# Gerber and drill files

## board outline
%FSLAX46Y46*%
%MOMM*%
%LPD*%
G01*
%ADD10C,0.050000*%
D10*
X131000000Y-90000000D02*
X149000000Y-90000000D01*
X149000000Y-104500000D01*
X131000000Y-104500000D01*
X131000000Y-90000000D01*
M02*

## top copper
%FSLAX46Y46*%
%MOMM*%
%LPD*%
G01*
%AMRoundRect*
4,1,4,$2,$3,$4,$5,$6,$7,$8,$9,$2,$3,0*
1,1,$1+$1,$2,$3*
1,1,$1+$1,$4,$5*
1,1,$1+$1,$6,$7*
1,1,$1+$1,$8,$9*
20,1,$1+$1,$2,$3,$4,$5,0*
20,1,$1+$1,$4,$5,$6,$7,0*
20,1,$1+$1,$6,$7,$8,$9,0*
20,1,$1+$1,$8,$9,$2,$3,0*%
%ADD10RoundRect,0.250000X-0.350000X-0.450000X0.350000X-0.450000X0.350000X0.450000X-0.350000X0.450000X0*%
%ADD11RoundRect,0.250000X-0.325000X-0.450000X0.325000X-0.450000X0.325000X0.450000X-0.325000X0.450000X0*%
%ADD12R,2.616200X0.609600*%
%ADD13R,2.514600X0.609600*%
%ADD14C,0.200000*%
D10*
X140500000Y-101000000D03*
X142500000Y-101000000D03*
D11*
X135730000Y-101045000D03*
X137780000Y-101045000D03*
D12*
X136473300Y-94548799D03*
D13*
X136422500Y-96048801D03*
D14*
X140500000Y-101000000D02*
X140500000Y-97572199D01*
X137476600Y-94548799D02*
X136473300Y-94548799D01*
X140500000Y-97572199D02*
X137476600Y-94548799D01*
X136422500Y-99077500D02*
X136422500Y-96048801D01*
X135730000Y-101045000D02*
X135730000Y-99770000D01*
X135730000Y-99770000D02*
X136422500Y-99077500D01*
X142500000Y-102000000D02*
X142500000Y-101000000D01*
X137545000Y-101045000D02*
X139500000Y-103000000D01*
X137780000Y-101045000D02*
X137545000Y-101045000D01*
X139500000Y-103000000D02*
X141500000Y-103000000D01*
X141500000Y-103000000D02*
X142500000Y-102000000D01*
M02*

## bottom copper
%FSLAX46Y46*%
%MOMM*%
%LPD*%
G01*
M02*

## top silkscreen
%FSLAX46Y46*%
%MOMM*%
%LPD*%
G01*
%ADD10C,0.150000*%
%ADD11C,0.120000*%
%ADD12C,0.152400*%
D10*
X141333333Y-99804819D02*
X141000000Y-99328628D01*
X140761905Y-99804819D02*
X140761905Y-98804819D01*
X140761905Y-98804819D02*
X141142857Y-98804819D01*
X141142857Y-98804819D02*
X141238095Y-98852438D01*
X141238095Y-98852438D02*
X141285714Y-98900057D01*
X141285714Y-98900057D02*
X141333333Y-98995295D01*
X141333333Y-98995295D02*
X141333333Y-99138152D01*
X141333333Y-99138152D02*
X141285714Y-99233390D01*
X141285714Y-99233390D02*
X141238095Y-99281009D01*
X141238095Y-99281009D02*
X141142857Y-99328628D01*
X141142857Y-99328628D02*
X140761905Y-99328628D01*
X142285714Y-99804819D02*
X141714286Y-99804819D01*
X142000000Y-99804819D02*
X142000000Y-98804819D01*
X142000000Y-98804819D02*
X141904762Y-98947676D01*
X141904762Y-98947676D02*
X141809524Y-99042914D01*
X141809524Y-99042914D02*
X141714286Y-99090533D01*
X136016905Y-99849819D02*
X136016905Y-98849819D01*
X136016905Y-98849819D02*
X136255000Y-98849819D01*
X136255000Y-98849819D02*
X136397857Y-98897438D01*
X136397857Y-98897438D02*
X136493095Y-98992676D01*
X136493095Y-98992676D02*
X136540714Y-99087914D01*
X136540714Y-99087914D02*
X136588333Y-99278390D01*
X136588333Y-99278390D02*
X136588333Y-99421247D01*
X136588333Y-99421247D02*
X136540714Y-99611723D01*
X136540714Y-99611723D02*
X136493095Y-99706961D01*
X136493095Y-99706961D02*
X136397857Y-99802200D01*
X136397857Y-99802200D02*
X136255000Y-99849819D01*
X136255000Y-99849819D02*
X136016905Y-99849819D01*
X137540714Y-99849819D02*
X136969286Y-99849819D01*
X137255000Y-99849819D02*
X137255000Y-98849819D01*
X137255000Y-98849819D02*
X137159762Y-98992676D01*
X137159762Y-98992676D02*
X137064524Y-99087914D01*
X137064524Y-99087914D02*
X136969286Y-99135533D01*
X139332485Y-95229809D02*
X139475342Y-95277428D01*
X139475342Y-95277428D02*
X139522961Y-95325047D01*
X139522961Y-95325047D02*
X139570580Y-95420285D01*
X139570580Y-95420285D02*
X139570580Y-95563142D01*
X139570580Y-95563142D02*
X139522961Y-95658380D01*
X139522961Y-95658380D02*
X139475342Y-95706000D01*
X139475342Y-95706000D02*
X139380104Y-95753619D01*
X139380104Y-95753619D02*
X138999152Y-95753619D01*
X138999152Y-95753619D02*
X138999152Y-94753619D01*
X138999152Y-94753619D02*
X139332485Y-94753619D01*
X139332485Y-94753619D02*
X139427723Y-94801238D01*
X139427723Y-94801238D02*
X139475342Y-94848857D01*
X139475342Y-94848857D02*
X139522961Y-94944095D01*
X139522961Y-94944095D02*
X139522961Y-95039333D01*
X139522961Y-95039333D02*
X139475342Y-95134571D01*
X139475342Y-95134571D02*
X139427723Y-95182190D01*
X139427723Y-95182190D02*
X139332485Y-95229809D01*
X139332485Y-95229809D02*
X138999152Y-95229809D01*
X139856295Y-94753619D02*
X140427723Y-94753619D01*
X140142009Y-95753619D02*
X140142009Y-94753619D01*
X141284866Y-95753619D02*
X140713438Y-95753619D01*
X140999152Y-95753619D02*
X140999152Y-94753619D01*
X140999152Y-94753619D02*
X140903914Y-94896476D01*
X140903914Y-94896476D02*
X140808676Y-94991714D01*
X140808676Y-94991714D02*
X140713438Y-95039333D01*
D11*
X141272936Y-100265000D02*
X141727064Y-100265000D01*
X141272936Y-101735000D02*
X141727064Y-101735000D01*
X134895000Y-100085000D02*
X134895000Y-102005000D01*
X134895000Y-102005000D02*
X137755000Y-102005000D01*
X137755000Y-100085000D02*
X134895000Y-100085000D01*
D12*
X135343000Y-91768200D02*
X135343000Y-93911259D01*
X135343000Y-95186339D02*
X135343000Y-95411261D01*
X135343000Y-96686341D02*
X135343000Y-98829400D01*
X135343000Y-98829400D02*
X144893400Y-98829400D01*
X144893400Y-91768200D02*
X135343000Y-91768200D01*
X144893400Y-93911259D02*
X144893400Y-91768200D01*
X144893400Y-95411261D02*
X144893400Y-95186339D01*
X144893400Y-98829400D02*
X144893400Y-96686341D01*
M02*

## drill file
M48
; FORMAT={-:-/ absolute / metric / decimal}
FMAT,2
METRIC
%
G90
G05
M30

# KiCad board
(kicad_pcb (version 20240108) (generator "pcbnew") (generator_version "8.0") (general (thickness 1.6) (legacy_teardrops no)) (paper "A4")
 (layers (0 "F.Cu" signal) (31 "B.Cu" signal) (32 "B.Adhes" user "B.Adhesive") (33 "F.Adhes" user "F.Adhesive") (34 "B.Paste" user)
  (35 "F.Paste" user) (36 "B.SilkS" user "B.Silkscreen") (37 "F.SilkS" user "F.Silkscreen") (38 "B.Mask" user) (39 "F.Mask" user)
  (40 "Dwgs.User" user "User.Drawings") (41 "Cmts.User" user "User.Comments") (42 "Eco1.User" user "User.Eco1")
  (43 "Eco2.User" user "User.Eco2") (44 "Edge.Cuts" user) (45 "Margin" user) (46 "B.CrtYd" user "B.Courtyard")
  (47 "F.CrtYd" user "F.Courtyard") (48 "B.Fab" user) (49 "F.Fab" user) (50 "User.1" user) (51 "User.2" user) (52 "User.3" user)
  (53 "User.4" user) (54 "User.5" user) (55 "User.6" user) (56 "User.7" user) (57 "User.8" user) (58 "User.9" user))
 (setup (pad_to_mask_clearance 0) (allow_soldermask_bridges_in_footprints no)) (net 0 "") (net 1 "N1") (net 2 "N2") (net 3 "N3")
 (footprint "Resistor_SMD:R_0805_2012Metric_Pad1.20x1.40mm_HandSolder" (layer "F.Cu") (at 141.5 101)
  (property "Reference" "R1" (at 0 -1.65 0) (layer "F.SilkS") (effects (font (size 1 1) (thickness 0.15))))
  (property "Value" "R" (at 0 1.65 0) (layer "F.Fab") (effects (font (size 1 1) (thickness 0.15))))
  (fp_line (start -0.227064 -0.735) (end 0.227064 -0.735) (stroke (width 0.12) (type solid)) (layer "F.SilkS"))
  (fp_line (start -0.227064 0.735) (end 0.227064 0.735) (stroke (width 0.12) (type solid)) (layer "F.SilkS"))
  (pad "1" smd roundrect (at -1 0) (size 1.2 1.4) (layers "F.Cu" "F.Paste" "F.Mask") (roundrect_rratio 0.208333) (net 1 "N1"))
  (pad "2" smd roundrect (at 1 0) (size 1.2 1.4) (layers "F.Cu" "F.Paste" "F.Mask") (roundrect_rratio 0.208333) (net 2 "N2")))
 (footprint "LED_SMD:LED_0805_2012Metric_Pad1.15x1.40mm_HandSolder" (layer "F.Cu") (at 136.755 101.045)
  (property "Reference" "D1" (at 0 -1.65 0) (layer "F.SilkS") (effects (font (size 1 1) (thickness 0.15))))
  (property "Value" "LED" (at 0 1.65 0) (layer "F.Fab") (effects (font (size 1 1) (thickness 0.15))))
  (fp_line (start -1.86 -0.96) (end -1.86 0.96) (stroke (width 0.12) (type solid)) (layer "F.SilkS"))
  (fp_line (start -1.86 0.96) (end 1 0.96) (stroke (width 0.12) (type solid)) (layer "F.SilkS"))
  (fp_line (start 1 -0.96) (end -1.86 -0.96) (stroke (width 0.12) (type solid)) (layer "F.SilkS"))
  (pad "1" smd roundrect (at -1.025 0) (size 1.15 1.4) (layers "F.Cu" "F.Paste" "F.Mask") (roundrect_rratio 0.217391) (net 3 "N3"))
  (pad "2" smd roundrect (at 1.025 0) (size 1.15 1.4) (layers "F.Cu" "F.Paste" "F.Mask") (roundrect_rratio 0.217391) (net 2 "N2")))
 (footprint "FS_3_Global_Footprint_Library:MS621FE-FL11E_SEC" (layer "F.Cu") (at 140.1182 95.2988)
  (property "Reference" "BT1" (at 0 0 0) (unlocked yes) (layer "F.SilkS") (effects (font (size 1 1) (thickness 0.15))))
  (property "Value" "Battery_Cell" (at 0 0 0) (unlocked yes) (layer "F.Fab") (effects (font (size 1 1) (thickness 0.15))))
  (fp_line (start -4.7752 -3.5306) (end -4.7752 -1.387541) (stroke (width 0.1524) (type solid)) (layer "F.SilkS"))
  (fp_line (start -4.7752 -0.112461) (end -4.7752 0.112461) (stroke (width 0.1524) (type solid)) (layer "F.SilkS"))
  (fp_line (start -4.7752 1.387541) (end -4.7752 3.5306) (stroke (width 0.1524) (type solid)) (layer "F.SilkS"))
  (fp_line (start -4.7752 3.5306) (end 4.7752 3.5306) (stroke (width 0.1524) (type solid)) (layer "F.SilkS"))
  (fp_line (start 4.7752 -3.5306) (end -4.7752 -3.5306) (stroke (width 0.1524) (type solid)) (layer "F.SilkS"))
  (fp_line (start 4.7752 -1.387541) (end 4.7752 -3.5306) (stroke (width 0.1524) (type solid)) (layer "F.SilkS"))
  (fp_line (start 4.7752 0.112461) (end 4.7752 -0.112461) (stroke (width 0.1524) (type solid)) (layer "F.SilkS"))
  (fp_line (start 4.7752 3.5306) (end 4.7752 1.387541) (stroke (width 0.1524) (type solid)) (layer "F.SilkS"))
  (pad "1" smd rect (at -3.6449 -0.750001) (size 2.6162 0.6096) (layers "F.Cu" "F.Paste" "F.Mask") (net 1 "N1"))
  (pad "2" smd rect (at -3.6957 0.750001) (size 2.5146 0.6096) (layers "F.Cu" "F.Paste" "F.Mask") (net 3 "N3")))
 (gr_rect (start 131 90) (end 149 104.5) (stroke (width 0.05) (type default)) (fill none) (layer "Edge.Cuts"))
 (segment (start 140.5 101) (end 140.5 97.572199) (width 0.2) (layer "F.Cu") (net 1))
 (segment (start 137.4766 94.548799) (end 136.4733 94.548799) (width 0.2) (layer "F.Cu") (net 1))
 (segment (start 140.5 97.572199) (end 137.4766 94.548799) (width 0.2) (layer "F.Cu") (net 1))
 (segment (start 136.4225 99.0775) (end 136.4225 96.048801) (width 0.2) (layer "F.Cu") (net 3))
 (segment (start 135.73 101.045) (end 135.73 99.77) (width 0.2) (layer "F.Cu") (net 3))
 (segment (start 135.73 99.77) (end 136.4225 99.0775) (width 0.2) (layer "F.Cu") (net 3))
 (segment (start 142.5 102) (end 142.5 101) (width 0.2) (layer "F.Cu") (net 2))
 (segment (start 137.545 101.045) (end 139.5 103) (width 0.2) (layer "F.Cu") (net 2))
 (segment (start 137.78 101.045) (end 137.545 101.045) (width 0.2) (layer "F.Cu") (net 2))
 (segment (start 139.5 103) (end 141.5 103) (width 0.2) (layer "F.Cu") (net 2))
 (segment (start 141.5 103) (end 142.5 102) (width 0.2) (layer "F.Cu") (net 2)))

